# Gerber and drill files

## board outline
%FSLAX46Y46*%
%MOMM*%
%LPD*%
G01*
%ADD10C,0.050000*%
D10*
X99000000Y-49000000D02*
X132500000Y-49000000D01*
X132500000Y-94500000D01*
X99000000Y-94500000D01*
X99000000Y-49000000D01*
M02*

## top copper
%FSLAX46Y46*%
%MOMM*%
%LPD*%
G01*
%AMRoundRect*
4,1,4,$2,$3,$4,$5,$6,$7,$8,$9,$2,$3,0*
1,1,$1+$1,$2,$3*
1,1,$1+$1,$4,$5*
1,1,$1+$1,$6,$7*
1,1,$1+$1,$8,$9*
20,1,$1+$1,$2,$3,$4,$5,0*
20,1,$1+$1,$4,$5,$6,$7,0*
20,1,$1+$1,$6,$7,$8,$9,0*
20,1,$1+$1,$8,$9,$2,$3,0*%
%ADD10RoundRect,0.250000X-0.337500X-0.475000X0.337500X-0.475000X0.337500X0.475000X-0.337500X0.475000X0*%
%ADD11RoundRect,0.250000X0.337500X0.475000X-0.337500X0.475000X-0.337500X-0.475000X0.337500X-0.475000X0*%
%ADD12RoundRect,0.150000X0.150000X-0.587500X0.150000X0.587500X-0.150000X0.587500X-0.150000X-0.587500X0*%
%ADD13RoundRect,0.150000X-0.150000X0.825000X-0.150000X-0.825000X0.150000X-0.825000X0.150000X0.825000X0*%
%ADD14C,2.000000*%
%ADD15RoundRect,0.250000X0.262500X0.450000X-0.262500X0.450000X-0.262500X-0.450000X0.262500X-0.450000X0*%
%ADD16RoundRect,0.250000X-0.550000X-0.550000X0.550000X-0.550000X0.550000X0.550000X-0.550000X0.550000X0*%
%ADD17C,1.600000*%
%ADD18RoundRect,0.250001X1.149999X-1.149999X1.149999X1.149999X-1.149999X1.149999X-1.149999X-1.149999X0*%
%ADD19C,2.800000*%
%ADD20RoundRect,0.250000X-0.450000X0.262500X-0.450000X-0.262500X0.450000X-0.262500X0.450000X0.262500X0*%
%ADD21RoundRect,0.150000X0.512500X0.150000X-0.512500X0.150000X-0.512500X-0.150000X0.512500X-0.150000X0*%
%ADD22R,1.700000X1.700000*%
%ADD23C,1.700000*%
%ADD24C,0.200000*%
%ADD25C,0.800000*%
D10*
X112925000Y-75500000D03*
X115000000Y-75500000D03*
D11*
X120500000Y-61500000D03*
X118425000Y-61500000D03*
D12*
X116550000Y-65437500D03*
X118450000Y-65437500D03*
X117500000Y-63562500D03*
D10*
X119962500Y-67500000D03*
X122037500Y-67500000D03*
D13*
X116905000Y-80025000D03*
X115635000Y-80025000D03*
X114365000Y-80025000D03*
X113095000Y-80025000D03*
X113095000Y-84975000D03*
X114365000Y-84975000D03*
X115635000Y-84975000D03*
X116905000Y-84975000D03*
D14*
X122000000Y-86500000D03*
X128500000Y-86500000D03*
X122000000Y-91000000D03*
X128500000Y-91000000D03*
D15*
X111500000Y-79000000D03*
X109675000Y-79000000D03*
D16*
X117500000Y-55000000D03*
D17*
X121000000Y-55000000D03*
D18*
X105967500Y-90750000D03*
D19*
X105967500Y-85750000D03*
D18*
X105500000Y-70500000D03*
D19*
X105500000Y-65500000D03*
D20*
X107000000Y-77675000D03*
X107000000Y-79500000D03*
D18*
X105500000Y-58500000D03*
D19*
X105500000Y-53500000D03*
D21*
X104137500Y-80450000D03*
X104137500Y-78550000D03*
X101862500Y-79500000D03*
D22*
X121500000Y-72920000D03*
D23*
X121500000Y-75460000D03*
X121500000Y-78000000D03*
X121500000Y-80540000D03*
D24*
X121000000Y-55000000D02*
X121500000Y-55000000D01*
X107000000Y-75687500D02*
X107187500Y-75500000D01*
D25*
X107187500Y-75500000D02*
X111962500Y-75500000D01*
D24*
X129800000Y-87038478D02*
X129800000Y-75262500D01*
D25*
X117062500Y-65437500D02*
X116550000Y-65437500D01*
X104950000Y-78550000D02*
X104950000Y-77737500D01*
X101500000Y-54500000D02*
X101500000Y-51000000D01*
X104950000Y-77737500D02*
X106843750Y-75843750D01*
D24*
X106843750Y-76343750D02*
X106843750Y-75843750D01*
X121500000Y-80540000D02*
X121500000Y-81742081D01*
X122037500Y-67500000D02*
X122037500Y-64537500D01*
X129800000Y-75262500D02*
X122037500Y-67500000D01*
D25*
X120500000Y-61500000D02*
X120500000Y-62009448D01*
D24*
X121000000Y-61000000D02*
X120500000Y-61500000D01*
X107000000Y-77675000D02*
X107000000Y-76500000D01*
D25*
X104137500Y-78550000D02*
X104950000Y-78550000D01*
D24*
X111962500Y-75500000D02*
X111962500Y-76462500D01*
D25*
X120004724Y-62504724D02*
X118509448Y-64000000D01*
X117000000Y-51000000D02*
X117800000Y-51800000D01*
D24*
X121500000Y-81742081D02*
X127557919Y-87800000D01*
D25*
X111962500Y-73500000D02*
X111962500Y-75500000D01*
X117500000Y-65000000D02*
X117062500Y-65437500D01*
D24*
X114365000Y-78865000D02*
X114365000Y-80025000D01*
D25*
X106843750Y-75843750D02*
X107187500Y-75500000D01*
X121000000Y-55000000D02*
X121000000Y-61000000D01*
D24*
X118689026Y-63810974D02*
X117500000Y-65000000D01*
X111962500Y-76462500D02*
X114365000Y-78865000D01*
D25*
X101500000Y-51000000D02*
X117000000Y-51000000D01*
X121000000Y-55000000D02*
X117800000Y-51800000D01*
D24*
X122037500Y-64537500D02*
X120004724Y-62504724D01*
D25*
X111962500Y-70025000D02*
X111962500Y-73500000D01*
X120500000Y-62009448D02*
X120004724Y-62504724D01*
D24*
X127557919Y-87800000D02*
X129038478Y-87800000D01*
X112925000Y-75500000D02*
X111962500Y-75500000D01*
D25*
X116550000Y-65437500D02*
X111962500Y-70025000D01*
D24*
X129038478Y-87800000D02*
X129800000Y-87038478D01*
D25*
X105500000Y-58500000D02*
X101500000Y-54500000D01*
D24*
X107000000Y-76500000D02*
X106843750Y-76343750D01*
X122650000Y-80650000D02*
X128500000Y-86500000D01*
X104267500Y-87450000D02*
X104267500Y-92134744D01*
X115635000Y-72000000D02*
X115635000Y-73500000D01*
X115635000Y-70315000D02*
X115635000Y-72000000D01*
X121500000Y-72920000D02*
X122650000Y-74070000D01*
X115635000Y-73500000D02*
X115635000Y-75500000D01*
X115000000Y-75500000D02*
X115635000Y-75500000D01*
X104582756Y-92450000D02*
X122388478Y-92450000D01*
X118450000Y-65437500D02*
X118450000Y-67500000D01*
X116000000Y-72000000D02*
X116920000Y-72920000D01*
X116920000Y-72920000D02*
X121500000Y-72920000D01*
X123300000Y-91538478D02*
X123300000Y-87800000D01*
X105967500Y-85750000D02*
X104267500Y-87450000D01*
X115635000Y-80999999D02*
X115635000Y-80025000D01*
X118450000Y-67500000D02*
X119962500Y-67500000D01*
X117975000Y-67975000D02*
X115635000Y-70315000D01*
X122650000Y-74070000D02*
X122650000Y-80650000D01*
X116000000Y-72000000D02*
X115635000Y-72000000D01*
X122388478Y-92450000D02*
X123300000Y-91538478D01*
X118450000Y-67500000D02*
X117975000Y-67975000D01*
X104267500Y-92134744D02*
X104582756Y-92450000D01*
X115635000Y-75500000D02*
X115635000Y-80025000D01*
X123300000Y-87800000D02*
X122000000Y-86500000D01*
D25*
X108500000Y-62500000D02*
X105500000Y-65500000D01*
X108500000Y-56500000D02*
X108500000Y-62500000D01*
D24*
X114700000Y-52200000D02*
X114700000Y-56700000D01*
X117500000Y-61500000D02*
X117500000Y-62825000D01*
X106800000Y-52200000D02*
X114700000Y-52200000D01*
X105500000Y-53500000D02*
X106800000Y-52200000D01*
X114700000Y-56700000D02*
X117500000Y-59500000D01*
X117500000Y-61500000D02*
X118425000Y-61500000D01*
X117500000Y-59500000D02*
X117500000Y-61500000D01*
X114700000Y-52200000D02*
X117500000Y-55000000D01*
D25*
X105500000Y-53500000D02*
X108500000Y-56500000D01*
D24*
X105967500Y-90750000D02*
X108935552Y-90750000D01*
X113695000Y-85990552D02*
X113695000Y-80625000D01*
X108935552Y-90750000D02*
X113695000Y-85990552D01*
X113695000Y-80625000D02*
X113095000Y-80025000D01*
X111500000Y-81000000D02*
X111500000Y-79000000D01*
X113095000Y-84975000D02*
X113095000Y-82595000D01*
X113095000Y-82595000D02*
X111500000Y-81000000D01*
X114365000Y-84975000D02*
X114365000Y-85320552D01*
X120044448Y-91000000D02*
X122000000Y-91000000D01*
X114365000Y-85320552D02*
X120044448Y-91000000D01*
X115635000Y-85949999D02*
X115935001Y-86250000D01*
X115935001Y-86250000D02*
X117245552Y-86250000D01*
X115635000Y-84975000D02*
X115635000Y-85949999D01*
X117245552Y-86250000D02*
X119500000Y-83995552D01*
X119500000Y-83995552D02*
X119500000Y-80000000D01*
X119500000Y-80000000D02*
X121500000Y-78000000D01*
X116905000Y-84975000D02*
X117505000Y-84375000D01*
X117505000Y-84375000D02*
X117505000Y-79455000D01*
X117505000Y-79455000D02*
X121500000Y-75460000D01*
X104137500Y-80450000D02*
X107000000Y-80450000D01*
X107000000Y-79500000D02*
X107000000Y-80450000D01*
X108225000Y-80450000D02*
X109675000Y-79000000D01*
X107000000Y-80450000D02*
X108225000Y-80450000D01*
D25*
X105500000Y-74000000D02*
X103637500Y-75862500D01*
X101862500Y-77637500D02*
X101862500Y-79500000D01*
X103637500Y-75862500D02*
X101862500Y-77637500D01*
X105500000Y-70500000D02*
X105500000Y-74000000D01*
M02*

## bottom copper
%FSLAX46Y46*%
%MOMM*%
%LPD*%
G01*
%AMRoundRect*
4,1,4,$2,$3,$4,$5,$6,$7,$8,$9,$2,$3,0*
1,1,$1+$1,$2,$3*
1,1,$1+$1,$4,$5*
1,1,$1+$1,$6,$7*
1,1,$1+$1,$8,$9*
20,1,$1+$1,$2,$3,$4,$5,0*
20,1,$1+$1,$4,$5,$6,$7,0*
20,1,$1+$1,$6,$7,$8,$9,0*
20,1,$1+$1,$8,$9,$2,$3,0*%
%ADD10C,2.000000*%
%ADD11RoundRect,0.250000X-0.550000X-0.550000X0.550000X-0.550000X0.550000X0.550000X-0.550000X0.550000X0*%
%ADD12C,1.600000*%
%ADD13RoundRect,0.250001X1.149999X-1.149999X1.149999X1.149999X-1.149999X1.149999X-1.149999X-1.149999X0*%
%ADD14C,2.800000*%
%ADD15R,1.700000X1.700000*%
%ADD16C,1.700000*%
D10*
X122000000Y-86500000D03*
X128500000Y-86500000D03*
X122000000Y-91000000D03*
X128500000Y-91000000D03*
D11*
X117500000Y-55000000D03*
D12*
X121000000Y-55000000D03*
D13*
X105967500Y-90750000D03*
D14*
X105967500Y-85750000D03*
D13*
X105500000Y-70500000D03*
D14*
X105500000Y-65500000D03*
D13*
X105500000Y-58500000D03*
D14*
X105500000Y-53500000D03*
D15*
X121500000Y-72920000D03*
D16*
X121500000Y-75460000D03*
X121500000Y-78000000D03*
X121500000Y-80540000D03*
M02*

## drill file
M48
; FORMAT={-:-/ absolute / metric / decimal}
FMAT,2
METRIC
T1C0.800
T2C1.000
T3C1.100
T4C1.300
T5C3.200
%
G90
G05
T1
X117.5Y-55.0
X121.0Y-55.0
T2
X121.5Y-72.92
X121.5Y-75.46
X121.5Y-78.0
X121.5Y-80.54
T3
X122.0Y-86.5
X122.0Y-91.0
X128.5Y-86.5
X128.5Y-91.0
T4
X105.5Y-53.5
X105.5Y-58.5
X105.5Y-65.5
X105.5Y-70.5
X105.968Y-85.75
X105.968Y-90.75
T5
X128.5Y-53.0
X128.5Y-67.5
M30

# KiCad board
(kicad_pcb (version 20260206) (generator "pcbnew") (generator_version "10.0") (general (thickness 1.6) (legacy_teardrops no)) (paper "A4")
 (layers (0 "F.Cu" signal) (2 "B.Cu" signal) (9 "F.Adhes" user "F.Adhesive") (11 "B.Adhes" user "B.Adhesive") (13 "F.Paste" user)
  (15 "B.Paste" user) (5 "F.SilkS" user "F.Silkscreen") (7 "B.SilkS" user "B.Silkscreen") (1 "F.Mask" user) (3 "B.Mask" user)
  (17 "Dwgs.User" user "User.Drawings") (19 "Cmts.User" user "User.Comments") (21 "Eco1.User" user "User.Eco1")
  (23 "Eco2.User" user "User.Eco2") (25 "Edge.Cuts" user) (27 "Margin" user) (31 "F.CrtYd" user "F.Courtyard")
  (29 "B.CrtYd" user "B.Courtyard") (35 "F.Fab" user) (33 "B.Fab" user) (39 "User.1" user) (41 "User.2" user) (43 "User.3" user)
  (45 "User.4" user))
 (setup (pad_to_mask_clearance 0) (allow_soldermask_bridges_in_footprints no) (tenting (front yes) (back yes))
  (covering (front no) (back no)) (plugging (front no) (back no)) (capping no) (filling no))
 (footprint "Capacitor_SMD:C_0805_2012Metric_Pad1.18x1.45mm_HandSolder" (layer "F.Cu") (at 113.9625 75.5)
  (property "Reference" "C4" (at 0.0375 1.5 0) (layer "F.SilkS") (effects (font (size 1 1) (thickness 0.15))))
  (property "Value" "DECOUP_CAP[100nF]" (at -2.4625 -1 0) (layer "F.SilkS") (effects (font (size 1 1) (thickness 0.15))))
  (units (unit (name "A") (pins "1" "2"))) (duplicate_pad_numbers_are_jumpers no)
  (pad "1" smd roundrect (at -1.0375 0) (size 1.175 1.45) (layers "F.Cu" "F.Mask" "F.Paste") (roundrect_rratio 0.212766) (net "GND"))
  (pad "2" smd roundrect (at 1.0375 0) (size 1.175 1.45) (layers "F.Cu" "F.Mask" "F.Paste") (roundrect_rratio 0.212766) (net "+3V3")))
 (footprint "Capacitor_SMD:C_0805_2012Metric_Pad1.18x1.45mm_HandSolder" (layer "F.Cu") (at 119.4625 61.5 180)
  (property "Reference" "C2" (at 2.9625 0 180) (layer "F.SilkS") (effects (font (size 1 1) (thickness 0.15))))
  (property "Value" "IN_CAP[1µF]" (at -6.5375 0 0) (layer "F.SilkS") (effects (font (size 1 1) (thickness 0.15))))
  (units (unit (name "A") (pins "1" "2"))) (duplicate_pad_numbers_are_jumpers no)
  (pad "1" smd roundrect (at -1.0375 0 180) (size 1.175 1.45) (layers "F.Cu" "F.Mask" "F.Paste") (roundrect_rratio 0.212766) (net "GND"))
  (pad "2" smd roundrect (at 1.0375 0 180) (size 1.175 1.45) (layers "F.Cu" "F.Mask" "F.Paste") (roundrect_rratio 0.212766) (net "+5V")))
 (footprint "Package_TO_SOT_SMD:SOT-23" (layer "F.Cu") (at 117.5 64.5 90)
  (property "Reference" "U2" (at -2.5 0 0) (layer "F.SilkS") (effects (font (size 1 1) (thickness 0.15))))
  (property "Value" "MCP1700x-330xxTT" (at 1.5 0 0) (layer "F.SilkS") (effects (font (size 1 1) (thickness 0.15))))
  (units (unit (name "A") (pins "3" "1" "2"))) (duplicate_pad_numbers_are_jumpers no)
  (pad "1" smd roundrect (at -0.9375 -0.95 90) (size 1.475 0.6) (layers "F.Cu" "F.Mask" "F.Paste") (roundrect_rratio 0.25) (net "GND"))
  (pad "2" smd roundrect (at -0.9375 0.95 90) (size 1.475 0.6) (layers "F.Cu" "F.Mask" "F.Paste") (roundrect_rratio 0.25) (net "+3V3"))
  (pad "3" smd roundrect (at 0.9375 0 90) (size 1.475 0.6) (layers "F.Cu" "F.Mask" "F.Paste") (roundrect_rratio 0.25) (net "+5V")))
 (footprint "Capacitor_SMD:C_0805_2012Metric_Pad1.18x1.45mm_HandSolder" (layer "F.Cu") (at 121 67.5)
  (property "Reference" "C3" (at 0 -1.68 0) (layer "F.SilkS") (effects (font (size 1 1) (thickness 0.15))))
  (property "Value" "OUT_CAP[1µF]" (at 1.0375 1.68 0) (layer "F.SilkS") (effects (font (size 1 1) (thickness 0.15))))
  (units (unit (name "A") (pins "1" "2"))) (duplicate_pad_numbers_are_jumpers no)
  (pad "1" smd roundrect (at -1.0375 0) (size 1.175 1.45) (layers "F.Cu" "F.Mask" "F.Paste") (roundrect_rratio 0.212766) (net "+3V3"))
  (pad "2" smd roundrect (at 1.0375 0) (size 1.175 1.45) (layers "F.Cu" "F.Mask" "F.Paste") (roundrect_rratio 0.212766) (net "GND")))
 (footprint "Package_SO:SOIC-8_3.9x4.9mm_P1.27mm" (layer "F.Cu") (at 115 82.5 -90)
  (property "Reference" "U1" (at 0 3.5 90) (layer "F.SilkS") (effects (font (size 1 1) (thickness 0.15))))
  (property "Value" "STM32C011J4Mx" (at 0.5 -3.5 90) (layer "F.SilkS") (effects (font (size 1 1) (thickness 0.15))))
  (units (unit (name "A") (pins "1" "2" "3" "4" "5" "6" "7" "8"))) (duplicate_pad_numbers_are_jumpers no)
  (pad "1" smd roundrect (at -2.475 -1.905 270) (size 1.95 0.6) (layers "F.Cu" "F.Mask" "F.Paste") (roundrect_rratio 0.25)
   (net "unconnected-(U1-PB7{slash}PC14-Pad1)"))
  (pad "2" smd roundrect (at -2.475 -0.635 270) (size 1.95 0.6) (layers "F.Cu" "F.Mask" "F.Paste") (roundrect_rratio 0.25) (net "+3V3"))
  (pad "3" smd roundrect (at -2.475 0.635 270) (size 1.95 0.6) (layers "F.Cu" "F.Mask" "F.Paste") (roundrect_rratio 0.25) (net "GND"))
  (pad "4" smd roundrect (at -2.475 1.905 270) (size 1.95 0.6) (layers "F.Cu" "F.Mask" "F.Paste") (roundrect_rratio 0.25)
   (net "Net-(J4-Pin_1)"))
  (pad "5" smd roundrect (at 2.475 1.905 270) (size 1.95 0.6) (layers "F.Cu" "F.Mask" "F.Paste") (roundrect_rratio 0.25)
   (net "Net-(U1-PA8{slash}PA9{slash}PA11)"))
  (pad "6" smd roundrect (at 2.475 0.635 270) (size 1.95 0.6) (layers "F.Cu" "F.Mask" "F.Paste") (roundrect_rratio 0.25)
   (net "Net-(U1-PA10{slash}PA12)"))
  (pad "7" smd roundrect (at 2.475 -0.635 270) (size 1.95 0.6) (layers "F.Cu" "F.Mask" "F.Paste") (roundrect_rratio 0.25)
   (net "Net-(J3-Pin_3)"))
  (pad "8" smd roundrect (at 2.475 -1.905 270) (size 1.95 0.6) (layers "F.Cu" "F.Mask" "F.Paste") (roundrect_rratio 0.25)
   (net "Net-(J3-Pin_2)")))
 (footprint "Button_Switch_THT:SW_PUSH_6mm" (layer "F.Cu") (at 122 86.5)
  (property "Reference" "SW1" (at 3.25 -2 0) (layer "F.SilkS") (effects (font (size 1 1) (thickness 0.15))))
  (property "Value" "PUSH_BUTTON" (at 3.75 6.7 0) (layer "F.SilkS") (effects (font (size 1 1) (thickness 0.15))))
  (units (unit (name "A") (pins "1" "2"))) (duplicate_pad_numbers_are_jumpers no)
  (pad "1" thru_hole circle (at 0 0 90) (size 2 2) (drill 1.1) (layers "*.Cu" "*.Mask") (remove_unused_layers no) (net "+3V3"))
  (pad "1" thru_hole circle (at 6.5 0 90) (size 2 2) (drill 1.1) (layers "*.Cu" "*.Mask") (remove_unused_layers no) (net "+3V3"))
  (pad "2" thru_hole circle (at 0 4.5 90) (size 2 2) (drill 1.1) (layers "*.Cu" "*.Mask") (remove_unused_layers no)
   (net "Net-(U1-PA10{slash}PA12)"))
  (pad "2" thru_hole circle (at 6.5 4.5 90) (size 2 2) (drill 1.1) (layers "*.Cu" "*.Mask") (remove_unused_layers no)
   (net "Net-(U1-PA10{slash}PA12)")))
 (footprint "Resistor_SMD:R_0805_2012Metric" (layer "F.Cu") (at 110.5875 79 180)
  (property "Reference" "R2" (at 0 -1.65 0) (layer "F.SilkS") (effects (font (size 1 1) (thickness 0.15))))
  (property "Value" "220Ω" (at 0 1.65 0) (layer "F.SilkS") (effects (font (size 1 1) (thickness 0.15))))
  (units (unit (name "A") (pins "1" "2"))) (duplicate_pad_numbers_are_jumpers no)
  (pad "1" smd roundrect (at -0.9125 0 180) (size 1.025 1.4) (layers "F.Cu" "F.Mask" "F.Paste") (roundrect_rratio 0.243902)
   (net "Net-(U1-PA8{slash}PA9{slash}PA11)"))
  (pad "2" smd roundrect (at 0.9125 0 180) (size 1.025 1.4) (layers "F.Cu" "F.Mask" "F.Paste") (roundrect_rratio 0.243902)
   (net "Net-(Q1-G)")))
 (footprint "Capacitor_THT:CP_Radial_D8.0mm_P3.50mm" (layer "F.Cu") (at 117.5 55)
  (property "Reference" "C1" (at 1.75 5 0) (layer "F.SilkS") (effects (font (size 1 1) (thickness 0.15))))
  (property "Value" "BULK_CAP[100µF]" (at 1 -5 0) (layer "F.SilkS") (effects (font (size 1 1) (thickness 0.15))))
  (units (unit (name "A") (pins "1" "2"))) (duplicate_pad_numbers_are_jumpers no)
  (pad "1" thru_hole roundrect (at 0 0) (size 1.6 1.6) (drill 0.8) (layers "*.Cu" "*.Mask") (remove_unused_layers no)
   (roundrect_rratio 0.15625) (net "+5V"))
  (pad "2" thru_hole circle (at 3.5 0) (size 1.6 1.6) (drill 0.8) (layers "*.Cu" "*.Mask") (remove_unused_layers no) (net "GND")))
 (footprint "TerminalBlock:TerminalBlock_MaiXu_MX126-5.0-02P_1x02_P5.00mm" (layer "F.Cu") (at 105.9675 90.75 90)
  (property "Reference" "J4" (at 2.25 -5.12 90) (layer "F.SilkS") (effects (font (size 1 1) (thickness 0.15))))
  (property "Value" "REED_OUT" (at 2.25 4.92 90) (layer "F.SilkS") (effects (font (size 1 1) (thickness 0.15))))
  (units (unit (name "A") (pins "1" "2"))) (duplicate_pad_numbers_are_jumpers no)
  (pad "1" thru_hole roundrect (at 0 0 90) (size 2.8 2.8) (drill 1.3) (layers "*.Cu" "*.Mask") (remove_unused_layers no)
   (roundrect_rratio 0.089286) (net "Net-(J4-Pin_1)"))
  (pad "2" thru_hole circle (at 5 0 90) (size 2.8 2.8) (drill 1.3) (layers "*.Cu" "*.Mask") (remove_unused_layers no) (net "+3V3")))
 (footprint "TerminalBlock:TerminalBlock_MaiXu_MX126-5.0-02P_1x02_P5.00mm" (layer "F.Cu") (at 105.5 70.5 90)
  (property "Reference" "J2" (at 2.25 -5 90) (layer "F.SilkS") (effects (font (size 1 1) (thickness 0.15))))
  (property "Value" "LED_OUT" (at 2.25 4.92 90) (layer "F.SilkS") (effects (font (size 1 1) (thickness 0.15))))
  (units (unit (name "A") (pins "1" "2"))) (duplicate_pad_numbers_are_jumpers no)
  (pad "1" thru_hole roundrect (at 0 0 90) (size 2.8 2.8) (drill 1.3) (layers "*.Cu" "*.Mask") (remove_unused_layers no)
   (roundrect_rratio 0.089286) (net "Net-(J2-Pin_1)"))
  (pad "2" thru_hole circle (at 5 0 90) (size 2.8 2.8) (drill 1.3) (layers "*.Cu" "*.Mask") (remove_unused_layers no) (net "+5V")))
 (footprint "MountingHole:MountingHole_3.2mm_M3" (layer "F.Cu") (at 128.5 67.5)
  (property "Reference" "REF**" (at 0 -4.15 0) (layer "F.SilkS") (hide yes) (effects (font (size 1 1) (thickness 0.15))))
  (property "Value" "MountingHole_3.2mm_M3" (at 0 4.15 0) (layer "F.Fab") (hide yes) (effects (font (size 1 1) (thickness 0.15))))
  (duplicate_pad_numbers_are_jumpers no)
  (pad "" np_thru_hole circle (at 0 0) (size 3.2 3.2) (drill 3.2) (layers "*.Cu" "*.Mask")))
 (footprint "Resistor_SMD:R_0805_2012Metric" (layer "F.Cu") (at 107 78.5875 -90)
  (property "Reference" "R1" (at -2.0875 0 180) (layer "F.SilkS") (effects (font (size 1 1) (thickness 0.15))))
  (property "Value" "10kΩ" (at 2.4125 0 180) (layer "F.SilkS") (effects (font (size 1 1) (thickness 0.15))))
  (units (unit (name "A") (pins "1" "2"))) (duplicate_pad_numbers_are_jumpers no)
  (pad "1" smd roundrect (at -0.9125 0 270) (size 1.025 1.4) (layers "F.Cu" "F.Mask" "F.Paste") (roundrect_rratio 0.243902) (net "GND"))
  (pad "2" smd roundrect (at 0.9125 0 270) (size 1.025 1.4) (layers "F.Cu" "F.Mask" "F.Paste") (roundrect_rratio 0.243902)
   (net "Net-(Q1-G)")))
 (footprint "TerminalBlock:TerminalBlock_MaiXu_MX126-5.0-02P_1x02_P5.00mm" (layer "F.Cu") (at 105.5 58.5 90)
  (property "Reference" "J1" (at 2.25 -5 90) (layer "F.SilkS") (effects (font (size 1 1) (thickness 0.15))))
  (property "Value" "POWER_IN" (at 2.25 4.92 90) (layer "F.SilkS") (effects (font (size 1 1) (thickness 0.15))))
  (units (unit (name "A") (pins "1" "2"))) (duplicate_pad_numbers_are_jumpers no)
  (pad "1" thru_hole roundrect (at 0 0 90) (size 2.8 2.8) (drill 1.3) (layers "*.Cu" "*.Mask") (remove_unused_layers no)
   (roundrect_rratio 0.089286) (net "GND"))
  (pad "2" thru_hole circle (at 5 0 90) (size 2.8 2.8) (drill 1.3) (layers "*.Cu" "*.Mask") (remove_unused_layers no) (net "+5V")))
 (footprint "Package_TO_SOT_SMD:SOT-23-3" (layer "F.Cu") (at 103 79.5 180)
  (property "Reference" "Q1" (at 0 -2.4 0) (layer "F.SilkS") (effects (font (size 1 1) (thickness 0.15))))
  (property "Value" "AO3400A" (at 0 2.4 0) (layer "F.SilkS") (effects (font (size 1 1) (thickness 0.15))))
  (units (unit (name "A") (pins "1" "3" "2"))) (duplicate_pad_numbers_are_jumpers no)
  (pad "1" smd roundrect (at -1.1375 -0.95 180) (size 1.325 0.6) (layers "F.Cu" "F.Mask" "F.Paste") (roundrect_rratio 0.25)
   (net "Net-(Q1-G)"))
  (pad "2" smd roundrect (at -1.1375 0.95 180) (size 1.325 0.6) (layers "F.Cu" "F.Mask" "F.Paste") (roundrect_rratio 0.25) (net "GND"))
  (pad "3" smd roundrect (at 1.1375 0 180) (size 1.325 0.6) (layers "F.Cu" "F.Mask" "F.Paste") (roundrect_rratio 0.25)
   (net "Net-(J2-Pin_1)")))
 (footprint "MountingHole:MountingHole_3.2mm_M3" (layer "F.Cu") (at 128.5 53)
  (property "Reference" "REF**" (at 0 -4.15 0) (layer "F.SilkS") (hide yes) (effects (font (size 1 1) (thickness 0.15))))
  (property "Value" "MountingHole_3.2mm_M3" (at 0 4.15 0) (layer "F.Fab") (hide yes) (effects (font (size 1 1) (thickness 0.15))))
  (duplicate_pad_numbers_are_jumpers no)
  (pad "" np_thru_hole circle (at 0 0) (size 3.2 3.2) (drill 3.2) (layers "*.Cu" "*.Mask")))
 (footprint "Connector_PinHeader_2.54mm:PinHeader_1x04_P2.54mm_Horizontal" (layer "F.Cu") (at 121.5 72.92)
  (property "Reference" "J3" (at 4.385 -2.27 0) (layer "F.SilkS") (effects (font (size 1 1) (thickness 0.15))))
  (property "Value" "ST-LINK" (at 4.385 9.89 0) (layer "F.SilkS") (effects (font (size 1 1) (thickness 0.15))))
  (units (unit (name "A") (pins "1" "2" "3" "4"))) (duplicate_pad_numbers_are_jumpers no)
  (pad "1" thru_hole rect (at 0 0) (size 1.7 1.7) (drill 1) (layers "*.Cu" "*.Mask") (remove_unused_layers no) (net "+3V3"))
  (pad "2" thru_hole circle (at 0 2.54) (size 1.7 1.7) (drill 1) (layers "*.Cu" "*.Mask") (remove_unused_layers no) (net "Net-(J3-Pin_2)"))
  (pad "3" thru_hole circle (at 0 5.08) (size 1.7 1.7) (drill 1) (layers "*.Cu" "*.Mask") (remove_unused_layers no) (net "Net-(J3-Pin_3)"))
  (pad "4" thru_hole circle (at 0 7.62) (size 1.7 1.7) (drill 1) (layers "*.Cu" "*.Mask") (remove_unused_layers no) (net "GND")))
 (gr_rect (start 99 49) (end 132.5 94.5) (stroke (width 0.05) (type default)) (fill no) (layer "Edge.Cuts"))
 (segment (start 121 55) (end 121.5 55) (width 0.2) (layer "F.Cu") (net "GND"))
 (segment (start 107 75.6875) (end 107.1875 75.5) (width 0.2) (layer "F.Cu") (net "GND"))
 (segment (start 107.1875 75.5) (end 111.9625 75.5) (width 0.8) (layer "F.Cu") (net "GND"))
 (segment (start 129.8 87.038478) (end 129.8 75.2625) (width 0.2) (layer "F.Cu") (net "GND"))
 (segment (start 117.0625 65.4375) (end 116.55 65.4375) (width 0.8) (layer "F.Cu") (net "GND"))
 (segment (start 104.95 78.55) (end 104.95 77.7375) (width 0.8) (layer "F.Cu") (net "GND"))
 (segment (start 101.5 54.5) (end 101.5 51) (width 0.8) (layer "F.Cu") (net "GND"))
 (segment (start 104.95 77.7375) (end 106.84375 75.84375) (width 0.8) (layer "F.Cu") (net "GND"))
 (segment (start 106.84375 76.34375) (end 106.84375 75.84375) (width 0.2) (layer "F.Cu") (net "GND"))
 (segment (start 121.5 80.54) (end 121.5 81.742081) (width 0.2) (layer "F.Cu") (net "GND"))
 (segment (start 122.0375 67.5) (end 122.0375 64.5375) (width 0.2) (layer "F.Cu") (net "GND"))
 (segment (start 129.8 75.2625) (end 122.0375 67.5) (width 0.2) (layer "F.Cu") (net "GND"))
 (segment (start 120.5 61.5) (end 120.5 62.009448) (width 0.8) (layer "F.Cu") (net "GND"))
 (segment (start 121 61) (end 120.5 61.5) (width 0.2) (layer "F.Cu") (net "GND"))
 (segment (start 107 77.675) (end 107 76.5) (width 0.2) (layer "F.Cu") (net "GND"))
 (segment (start 104.1375 78.55) (end 104.95 78.55) (width 0.8) (layer "F.Cu") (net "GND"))
 (segment (start 111.9625 75.5) (end 111.9625 76.4625) (width 0.2) (layer "F.Cu") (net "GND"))
 (segment (start 120.004724 62.504724) (end 118.509448 64) (width 0.8) (layer "F.Cu") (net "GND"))
 (segment (start 117 51) (end 117.8 51.8) (width 0.8) (layer "F.Cu") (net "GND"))
 (segment (start 121.5 81.742081) (end 127.557919 87.8) (width 0.2) (layer "F.Cu") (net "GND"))
 (segment (start 111.9625 73.5) (end 111.9625 75.5) (width 0.8) (layer "F.Cu") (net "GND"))
 (segment (start 117.5 65) (end 117.0625 65.4375) (width 0.8) (layer "F.Cu") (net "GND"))
 (segment (start 114.365 78.865) (end 114.365 80.025) (width 0.2) (layer "F.Cu") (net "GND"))
 (segment (start 106.84375 75.84375) (end 107.1875 75.5) (width 0.8) (layer "F.Cu") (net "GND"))
 (segment (start 121 55) (end 121 61) (width 0.8) (layer "F.Cu") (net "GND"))
 (segment (start 118.689026 63.810974) (end 117.5 65) (width 0.2) (layer "F.Cu") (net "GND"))
 (segment (start 111.9625 76.4625) (end 114.365 78.865) (width 0.2) (layer "F.Cu") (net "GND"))
 (segment (start 101.5 51) (end 117 51) (width 0.8) (layer "F.Cu") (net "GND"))
 (segment (start 121 55) (end 117.8 51.8) (width 0.8) (layer "F.Cu") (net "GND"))
 (segment (start 122.0375 64.5375) (end 120.004724 62.504724) (width 0.2) (layer "F.Cu") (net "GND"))
 (segment (start 111.9625 70.025) (end 111.9625 73.5) (width 0.8) (layer "F.Cu") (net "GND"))
 (segment (start 120.5 62.009448) (end 120.004724 62.504724) (width 0.8) (layer "F.Cu") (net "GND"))
 (segment (start 127.557919 87.8) (end 129.038478 87.8) (width 0.2) (layer "F.Cu") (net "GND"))
 (segment (start 112.925 75.5) (end 111.9625 75.5) (width 0.2) (layer "F.Cu") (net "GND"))
 (segment (start 116.55 65.4375) (end 111.9625 70.025) (width 0.8) (layer "F.Cu") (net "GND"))
 (segment (start 129.038478 87.8) (end 129.8 87.038478) (width 0.2) (layer "F.Cu") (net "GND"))
 (segment (start 105.5 58.5) (end 101.5 54.5) (width 0.8) (layer "F.Cu") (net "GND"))
 (segment (start 107 76.5) (end 106.84375 76.34375) (width 0.2) (layer "F.Cu") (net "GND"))
 (segment (start 122.65 80.65) (end 128.5 86.5) (width 0.2) (layer "F.Cu") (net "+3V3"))
 (segment (start 104.2675 87.45) (end 104.2675 92.134744) (width 0.2) (layer "F.Cu") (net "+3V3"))
 (segment (start 115.635 72) (end 115.635 73.5) (width 0.2) (layer "F.Cu") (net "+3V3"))
 (segment (start 115.635 70.315) (end 115.635 72) (width 0.2) (layer "F.Cu") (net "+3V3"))
 (segment (start 121.5 72.92) (end 122.65 74.07) (width 0.2) (layer "F.Cu") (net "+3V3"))
 (segment (start 115.635 73.5) (end 115.635 75.5) (width 0.2) (layer "F.Cu") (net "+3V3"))
 (segment (start 115 75.5) (end 115.635 75.5) (width 0.2) (layer "F.Cu") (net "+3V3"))
 (segment (start 104.582756 92.45) (end 122.388478 92.45) (width 0.2) (layer "F.Cu") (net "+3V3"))
 (segment (start 118.45 65.4375) (end 118.45 67.5) (width 0.2) (layer "F.Cu") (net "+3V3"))
 (segment (start 116 72) (end 116.92 72.92) (width 0.2) (layer "F.Cu") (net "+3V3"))
 (segment (start 116.92 72.92) (end 121.5 72.92) (width 0.2) (layer "F.Cu") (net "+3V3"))
 (segment (start 123.3 91.538478) (end 123.3 87.8) (width 0.2) (layer "F.Cu") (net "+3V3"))
 (segment (start 105.9675 85.75) (end 104.2675 87.45) (width 0.2) (layer "F.Cu") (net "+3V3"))
 (segment (start 115.635 80.999999) (end 115.635 80.025) (width 0.2) (layer "F.Cu") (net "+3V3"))
 (segment (start 118.45 67.5) (end 119.9625 67.5) (width 0.2) (layer "F.Cu") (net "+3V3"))
 (segment (start 117.975 67.975) (end 115.635 70.315) (width 0.2) (layer "F.Cu") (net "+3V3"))
 (segment (start 122.65 74.07) (end 122.65 80.65) (width 0.2) (layer "F.Cu") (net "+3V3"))
 (segment (start 116 72) (end 115.635 72) (width 0.2) (layer "F.Cu") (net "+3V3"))
 (segment (start 122.388478 92.45) (end 123.3 91.538478) (width 0.2) (layer "F.Cu") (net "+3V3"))
 (segment (start 118.45 67.5) (end 117.975 67.975) (width 0.2) (layer "F.Cu") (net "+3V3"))
 (segment (start 104.2675 92.134744) (end 104.582756 92.45) (width 0.2) (layer "F.Cu") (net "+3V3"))
 (segment (start 115.635 75.5) (end 115.635 80.025) (width 0.2) (layer "F.Cu") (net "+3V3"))
 (segment (start 123.3 87.8) (end 122 86.5) (width 0.2) (layer "F.Cu") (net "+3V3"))
 (segment (start 108.5 62.5) (end 105.5 65.5) (width 0.8) (layer "F.Cu") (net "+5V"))
 (segment (start 108.5 56.5) (end 108.5 62.5) (width 0.8) (layer "F.Cu") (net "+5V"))
 (segment (start 114.7 52.2) (end 114.7 56.7) (width 0.2) (layer "F.Cu") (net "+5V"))
 (segment (start 117.5 61.5) (end 117.5 62.825) (width 0.2) (layer "F.Cu") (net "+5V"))
 (segment (start 106.8 52.2) (end 114.7 52.2) (width 0.2) (layer "F.Cu") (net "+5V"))
 (segment (start 105.5 53.5) (end 106.8 52.2) (width 0.2) (layer "F.Cu") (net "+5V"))
 (segment (start 114.7 56.7) (end 117.5 59.5) (width 0.2) (layer "F.Cu") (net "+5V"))
 (segment (start 117.5 61.5) (end 118.425 61.5) (width 0.2) (layer "F.Cu") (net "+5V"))
 (segment (start 117.5 59.5) (end 117.5 61.5) (width 0.2) (layer "F.Cu") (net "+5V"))
 (segment (start 114.7 52.2) (end 117.5 55) (width 0.2) (layer "F.Cu") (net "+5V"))
 (segment (start 105.5 53.5) (end 108.5 56.5) (width 0.8) (layer "F.Cu") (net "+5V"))
 (segment (start 105.9675 90.75) (end 108.935552 90.75) (width 0.2) (layer "F.Cu") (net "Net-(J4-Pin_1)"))
 (segment (start 113.695 85.990552) (end 113.695 80.625) (width 0.2) (layer "F.Cu") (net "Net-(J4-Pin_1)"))
 (segment (start 108.935552 90.75) (end 113.695 85.990552) (width 0.2) (layer "F.Cu") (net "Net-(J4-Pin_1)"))
 (segment (start 113.695 80.625) (end 113.095 80.025) (width 0.2) (layer "F.Cu") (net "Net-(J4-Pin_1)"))
 (segment (start 111.5 81) (end 111.5 79) (width 0.2) (layer "F.Cu") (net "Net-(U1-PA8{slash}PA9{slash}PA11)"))
 (segment (start 113.095 84.975) (end 113.095 82.595) (width 0.2) (layer "F.Cu") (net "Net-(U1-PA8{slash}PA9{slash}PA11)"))
 (segment (start 113.095 82.595) (end 111.5 81) (width 0.2) (layer "F.Cu") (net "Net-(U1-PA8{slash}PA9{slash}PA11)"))
 (segment (start 114.365 84.975) (end 114.365 85.320552) (width 0.2) (layer "F.Cu") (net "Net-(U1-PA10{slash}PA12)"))
 (segment (start 120.044448 91) (end 122 91) (width 0.2) (layer "F.Cu") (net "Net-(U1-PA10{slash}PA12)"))
 (segment (start 114.365 85.320552) (end 120.044448 91) (width 0.2) (layer "F.Cu") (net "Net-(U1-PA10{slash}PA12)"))
 (segment (start 115.635 85.949999) (end 115.935001 86.25) (width 0.2) (layer "F.Cu") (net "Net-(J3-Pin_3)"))
 (segment (start 115.935001 86.25) (end 117.245552 86.25) (width 0.2) (layer "F.Cu") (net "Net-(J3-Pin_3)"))
 (segment (start 115.635 84.975) (end 115.635 85.949999) (width 0.2) (layer "F.Cu") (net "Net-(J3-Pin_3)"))
 (segment (start 117.245552 86.25) (end 119.5 83.995552) (width 0.2) (layer "F.Cu") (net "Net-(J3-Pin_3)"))
 (segment (start 119.5 83.995552) (end 119.5 80) (width 0.2) (layer "F.Cu") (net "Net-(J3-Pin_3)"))
 (segment (start 119.5 80) (end 121.5 78) (width 0.2) (layer "F.Cu") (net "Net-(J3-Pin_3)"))
 (segment (start 116.905 84.975) (end 117.505 84.375) (width 0.2) (layer "F.Cu") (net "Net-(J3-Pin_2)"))
 (segment (start 117.505 84.375) (end 117.505 79.455) (width 0.2) (layer "F.Cu") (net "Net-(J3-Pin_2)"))
 (segment (start 117.505 79.455) (end 121.5 75.46) (width 0.2) (layer "F.Cu") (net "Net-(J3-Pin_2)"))
 (segment (start 104.1375 80.45) (end 107 80.45) (width 0.2) (layer "F.Cu") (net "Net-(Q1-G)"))
 (segment (start 107 79.5) (end 107 80.45) (width 0.2) (layer "F.Cu") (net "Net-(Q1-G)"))
 (segment (start 108.225 80.45) (end 109.675 79) (width 0.2) (layer "F.Cu") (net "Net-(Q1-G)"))
 (segment (start 107 80.45) (end 108.225 80.45) (width 0.2) (layer "F.Cu") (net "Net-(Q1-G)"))
 (segment (start 105.5 74) (end 103.6375 75.8625) (width 0.8) (layer "F.Cu") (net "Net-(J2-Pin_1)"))
 (segment (start 101.8625 77.6375) (end 101.8625 79.5) (width 0.8) (layer "F.Cu") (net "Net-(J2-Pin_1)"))
 (segment (start 103.6375 75.8625) (end 101.8625 77.6375) (width 0.8) (layer "F.Cu") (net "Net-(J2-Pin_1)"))
 (segment (start 105.5 70.5) (end 105.5 74) (width 0.8) (layer "F.Cu") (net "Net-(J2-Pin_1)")))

